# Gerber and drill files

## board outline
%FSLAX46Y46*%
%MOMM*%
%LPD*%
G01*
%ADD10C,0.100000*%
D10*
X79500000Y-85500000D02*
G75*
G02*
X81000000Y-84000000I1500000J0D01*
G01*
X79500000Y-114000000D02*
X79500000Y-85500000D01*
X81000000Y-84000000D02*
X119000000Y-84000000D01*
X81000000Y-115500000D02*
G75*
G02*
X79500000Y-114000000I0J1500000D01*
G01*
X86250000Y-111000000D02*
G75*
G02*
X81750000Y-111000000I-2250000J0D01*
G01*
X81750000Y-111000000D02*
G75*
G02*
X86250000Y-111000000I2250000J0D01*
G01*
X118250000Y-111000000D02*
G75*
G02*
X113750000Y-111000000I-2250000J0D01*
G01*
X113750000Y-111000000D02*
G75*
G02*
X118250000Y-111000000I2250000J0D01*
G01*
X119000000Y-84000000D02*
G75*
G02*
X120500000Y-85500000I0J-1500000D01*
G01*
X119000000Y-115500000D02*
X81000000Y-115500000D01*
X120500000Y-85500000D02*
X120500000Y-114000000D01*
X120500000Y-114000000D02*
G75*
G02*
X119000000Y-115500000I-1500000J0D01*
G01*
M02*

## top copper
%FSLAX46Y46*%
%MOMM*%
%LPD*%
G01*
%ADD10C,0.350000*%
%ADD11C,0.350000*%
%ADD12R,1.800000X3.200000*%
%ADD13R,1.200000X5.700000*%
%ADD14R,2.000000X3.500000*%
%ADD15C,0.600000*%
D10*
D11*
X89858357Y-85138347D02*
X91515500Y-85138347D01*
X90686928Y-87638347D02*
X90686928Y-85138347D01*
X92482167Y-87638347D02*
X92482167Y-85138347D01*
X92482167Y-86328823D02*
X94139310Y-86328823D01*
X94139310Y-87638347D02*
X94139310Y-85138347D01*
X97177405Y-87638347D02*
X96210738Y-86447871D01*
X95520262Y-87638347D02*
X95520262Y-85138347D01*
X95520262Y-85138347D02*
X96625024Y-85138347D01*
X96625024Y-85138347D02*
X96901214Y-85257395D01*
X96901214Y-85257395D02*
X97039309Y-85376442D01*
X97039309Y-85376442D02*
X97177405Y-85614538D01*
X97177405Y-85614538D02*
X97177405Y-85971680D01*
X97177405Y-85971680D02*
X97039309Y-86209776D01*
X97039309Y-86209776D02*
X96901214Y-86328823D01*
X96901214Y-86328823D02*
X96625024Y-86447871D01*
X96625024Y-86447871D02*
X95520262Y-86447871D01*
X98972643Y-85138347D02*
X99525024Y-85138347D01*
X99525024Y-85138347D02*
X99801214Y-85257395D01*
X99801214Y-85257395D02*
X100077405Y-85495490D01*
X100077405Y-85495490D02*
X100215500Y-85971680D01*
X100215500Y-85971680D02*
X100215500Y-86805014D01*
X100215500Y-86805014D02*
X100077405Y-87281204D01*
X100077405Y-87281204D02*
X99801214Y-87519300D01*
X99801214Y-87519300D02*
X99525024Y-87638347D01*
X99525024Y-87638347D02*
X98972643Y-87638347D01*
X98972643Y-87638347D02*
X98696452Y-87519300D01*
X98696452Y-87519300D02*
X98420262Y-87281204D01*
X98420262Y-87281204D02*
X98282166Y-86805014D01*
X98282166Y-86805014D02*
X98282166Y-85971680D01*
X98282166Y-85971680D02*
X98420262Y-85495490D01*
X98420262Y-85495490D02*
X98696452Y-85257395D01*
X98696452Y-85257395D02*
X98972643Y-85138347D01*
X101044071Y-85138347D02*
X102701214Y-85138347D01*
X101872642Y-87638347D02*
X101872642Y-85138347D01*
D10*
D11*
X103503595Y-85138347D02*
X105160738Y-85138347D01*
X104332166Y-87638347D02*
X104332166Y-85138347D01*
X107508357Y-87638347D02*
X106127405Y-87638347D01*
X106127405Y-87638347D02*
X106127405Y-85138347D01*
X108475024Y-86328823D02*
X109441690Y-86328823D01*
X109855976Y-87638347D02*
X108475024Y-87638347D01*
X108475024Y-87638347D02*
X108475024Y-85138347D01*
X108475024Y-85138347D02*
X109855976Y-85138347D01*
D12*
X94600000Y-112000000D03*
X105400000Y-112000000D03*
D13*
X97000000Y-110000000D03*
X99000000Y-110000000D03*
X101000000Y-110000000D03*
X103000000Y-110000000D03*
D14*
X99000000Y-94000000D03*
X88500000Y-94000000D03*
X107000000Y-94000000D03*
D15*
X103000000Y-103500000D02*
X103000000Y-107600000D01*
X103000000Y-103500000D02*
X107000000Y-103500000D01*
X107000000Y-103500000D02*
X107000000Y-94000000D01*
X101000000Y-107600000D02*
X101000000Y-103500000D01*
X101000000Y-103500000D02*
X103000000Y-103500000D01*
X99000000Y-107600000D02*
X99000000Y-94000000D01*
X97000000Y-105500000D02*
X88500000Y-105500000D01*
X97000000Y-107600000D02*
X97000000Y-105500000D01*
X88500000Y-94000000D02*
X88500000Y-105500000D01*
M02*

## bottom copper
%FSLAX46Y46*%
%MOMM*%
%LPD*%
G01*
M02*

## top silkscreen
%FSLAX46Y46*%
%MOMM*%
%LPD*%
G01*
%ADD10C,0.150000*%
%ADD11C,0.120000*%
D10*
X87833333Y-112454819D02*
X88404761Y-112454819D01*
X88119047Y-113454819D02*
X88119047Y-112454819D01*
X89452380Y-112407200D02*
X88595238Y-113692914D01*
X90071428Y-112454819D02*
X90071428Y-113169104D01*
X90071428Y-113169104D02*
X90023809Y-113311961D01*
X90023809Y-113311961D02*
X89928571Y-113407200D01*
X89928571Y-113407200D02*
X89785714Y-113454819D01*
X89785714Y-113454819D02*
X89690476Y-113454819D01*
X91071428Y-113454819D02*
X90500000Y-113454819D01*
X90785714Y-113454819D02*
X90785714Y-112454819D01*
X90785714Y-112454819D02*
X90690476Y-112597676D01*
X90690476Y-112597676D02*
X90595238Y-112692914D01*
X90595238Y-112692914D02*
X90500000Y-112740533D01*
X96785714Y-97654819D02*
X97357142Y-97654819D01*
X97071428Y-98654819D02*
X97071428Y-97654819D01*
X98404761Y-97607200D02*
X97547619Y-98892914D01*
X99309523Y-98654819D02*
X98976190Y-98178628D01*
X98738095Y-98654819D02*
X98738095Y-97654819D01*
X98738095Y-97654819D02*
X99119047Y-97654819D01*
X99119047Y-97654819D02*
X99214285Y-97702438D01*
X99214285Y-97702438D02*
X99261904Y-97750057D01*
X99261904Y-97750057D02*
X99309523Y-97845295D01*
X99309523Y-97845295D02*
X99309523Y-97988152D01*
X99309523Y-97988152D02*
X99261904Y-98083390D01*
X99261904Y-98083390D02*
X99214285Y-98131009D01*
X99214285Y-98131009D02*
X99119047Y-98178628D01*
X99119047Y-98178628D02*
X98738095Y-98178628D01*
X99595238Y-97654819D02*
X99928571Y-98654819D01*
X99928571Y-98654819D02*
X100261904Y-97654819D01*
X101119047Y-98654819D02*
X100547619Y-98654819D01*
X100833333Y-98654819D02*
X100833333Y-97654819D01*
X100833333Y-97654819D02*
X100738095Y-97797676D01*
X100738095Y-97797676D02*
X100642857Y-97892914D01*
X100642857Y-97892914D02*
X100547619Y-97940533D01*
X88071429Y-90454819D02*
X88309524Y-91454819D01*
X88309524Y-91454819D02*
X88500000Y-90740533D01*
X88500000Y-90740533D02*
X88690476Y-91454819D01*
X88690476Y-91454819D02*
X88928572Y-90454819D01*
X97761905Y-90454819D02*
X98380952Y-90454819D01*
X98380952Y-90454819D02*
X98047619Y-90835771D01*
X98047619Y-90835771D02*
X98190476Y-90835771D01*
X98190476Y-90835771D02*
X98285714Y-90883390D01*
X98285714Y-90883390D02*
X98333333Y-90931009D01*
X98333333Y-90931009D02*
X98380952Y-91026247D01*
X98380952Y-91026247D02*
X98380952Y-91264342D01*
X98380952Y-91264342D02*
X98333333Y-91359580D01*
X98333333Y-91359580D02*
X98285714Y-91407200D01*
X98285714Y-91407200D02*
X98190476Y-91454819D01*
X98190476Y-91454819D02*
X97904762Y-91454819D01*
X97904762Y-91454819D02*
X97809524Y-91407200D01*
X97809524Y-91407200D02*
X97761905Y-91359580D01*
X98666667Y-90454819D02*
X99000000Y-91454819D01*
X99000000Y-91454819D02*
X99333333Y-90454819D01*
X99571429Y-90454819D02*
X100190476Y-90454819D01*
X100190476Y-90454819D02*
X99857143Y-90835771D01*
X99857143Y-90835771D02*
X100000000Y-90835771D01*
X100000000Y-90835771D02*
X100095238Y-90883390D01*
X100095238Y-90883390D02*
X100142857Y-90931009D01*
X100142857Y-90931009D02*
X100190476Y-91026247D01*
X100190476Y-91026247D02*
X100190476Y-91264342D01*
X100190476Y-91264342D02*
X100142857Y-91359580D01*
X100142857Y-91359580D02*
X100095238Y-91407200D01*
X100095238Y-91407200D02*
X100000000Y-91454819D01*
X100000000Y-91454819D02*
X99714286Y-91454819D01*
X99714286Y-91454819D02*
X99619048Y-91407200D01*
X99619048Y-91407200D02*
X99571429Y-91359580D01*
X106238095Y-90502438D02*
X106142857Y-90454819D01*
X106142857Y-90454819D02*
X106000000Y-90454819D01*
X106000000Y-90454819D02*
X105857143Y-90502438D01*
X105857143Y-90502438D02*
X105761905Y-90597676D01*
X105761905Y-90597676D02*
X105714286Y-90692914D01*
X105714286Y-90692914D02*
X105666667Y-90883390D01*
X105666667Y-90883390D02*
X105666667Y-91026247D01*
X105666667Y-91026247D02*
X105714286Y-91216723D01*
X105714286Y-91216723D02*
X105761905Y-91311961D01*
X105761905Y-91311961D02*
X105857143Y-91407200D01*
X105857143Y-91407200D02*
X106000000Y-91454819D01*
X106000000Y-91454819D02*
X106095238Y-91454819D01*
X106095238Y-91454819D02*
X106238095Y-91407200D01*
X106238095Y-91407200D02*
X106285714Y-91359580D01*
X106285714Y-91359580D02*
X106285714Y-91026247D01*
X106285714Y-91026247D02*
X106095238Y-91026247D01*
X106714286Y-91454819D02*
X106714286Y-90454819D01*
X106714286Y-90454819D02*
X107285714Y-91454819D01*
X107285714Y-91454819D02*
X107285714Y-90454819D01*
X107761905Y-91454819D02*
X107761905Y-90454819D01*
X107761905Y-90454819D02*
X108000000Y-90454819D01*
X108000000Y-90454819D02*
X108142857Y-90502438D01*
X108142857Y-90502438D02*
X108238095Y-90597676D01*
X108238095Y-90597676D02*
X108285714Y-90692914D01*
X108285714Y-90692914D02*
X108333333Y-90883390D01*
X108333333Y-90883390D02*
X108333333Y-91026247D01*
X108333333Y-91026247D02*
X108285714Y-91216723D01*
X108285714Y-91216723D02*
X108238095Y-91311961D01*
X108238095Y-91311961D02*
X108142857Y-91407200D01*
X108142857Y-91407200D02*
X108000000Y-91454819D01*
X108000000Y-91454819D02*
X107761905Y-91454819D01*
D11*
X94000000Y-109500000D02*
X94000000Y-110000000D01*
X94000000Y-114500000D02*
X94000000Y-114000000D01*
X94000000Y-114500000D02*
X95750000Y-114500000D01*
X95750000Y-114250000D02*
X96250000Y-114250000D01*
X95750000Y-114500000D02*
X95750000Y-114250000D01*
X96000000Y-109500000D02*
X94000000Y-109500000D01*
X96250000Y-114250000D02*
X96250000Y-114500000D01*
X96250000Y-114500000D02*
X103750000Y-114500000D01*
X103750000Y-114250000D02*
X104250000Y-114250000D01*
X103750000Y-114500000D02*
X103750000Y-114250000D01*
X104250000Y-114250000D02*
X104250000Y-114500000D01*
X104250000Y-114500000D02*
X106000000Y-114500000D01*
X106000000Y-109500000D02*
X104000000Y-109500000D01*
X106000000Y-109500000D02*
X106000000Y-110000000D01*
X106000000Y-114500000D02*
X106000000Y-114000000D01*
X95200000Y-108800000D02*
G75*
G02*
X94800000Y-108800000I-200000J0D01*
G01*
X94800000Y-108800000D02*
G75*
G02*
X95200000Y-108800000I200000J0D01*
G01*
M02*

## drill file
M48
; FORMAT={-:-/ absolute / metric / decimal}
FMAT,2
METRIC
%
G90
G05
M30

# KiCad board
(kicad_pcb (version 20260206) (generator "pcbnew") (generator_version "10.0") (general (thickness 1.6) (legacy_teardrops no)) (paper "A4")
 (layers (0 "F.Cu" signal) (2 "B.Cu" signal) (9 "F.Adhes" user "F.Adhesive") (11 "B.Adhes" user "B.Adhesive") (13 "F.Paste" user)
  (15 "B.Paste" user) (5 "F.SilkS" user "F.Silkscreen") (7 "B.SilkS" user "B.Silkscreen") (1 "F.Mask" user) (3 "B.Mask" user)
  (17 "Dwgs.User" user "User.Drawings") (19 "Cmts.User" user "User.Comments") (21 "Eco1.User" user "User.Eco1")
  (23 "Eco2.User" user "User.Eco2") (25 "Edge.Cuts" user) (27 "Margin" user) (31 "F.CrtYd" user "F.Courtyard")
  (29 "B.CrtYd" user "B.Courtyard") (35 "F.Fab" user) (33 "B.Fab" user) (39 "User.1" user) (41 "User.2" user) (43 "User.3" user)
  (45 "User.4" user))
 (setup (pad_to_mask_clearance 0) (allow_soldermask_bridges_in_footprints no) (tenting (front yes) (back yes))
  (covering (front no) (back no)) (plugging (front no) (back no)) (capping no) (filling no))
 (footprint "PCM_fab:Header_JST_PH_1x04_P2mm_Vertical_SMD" (layer "F.Cu") (at 98 110 90)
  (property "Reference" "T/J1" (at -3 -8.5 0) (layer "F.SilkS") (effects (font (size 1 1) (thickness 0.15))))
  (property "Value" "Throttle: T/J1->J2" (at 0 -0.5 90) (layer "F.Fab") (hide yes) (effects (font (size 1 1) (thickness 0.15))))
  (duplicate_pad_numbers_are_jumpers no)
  (fp_line (start 0.5 -4) (end 0 -4) (stroke (width 0.12) (type solid)) (layer "F.SilkS"))
  (fp_line (start -4.5 -4) (end -4 -4) (stroke (width 0.12) (type solid)) (layer "F.SilkS"))
  (fp_line (start -4.5 -4) (end -4.5 -2.25) (stroke (width 0.12) (type solid)) (layer "F.SilkS"))
  (fp_line (start -4.25 -2.25) (end -4.25 -1.75) (stroke (width 0.12) (type solid)) (layer "F.SilkS"))
  (fp_line (start -4.5 -2.25) (end -4.25 -2.25) (stroke (width 0.12) (type solid)) (layer "F.SilkS"))
  (fp_line (start 0.5 -2) (end 0.5 -4) (stroke (width 0.12) (type solid)) (layer "F.SilkS"))
  (fp_line (start -4.25 -1.75) (end -4.5 -1.75) (stroke (width 0.12) (type solid)) (layer "F.SilkS"))
  (fp_line (start -4.5 -1.75) (end -4.5 5.75) (stroke (width 0.12) (type solid)) (layer "F.SilkS"))
  (fp_line (start -4.25 5.75) (end -4.25 6.25) (stroke (width 0.12) (type solid)) (layer "F.SilkS"))
  (fp_line (start -4.5 5.75) (end -4.25 5.75) (stroke (width 0.12) (type solid)) (layer "F.SilkS"))
  (fp_line (start -4.25 6.25) (end -4.5 6.25) (stroke (width 0.12) (type solid)) (layer "F.SilkS"))
  (fp_line (start -4.5 6.25) (end -4.5 8) (stroke (width 0.12) (type solid)) (layer "F.SilkS"))
  (fp_line (start 0.5 8) (end 0.5 6) (stroke (width 0.12) (type solid)) (layer "F.SilkS"))
  (fp_line (start 0.5 8) (end 0 8) (stroke (width 0.12) (type solid)) (layer "F.SilkS"))
  (fp_line (start -4.5 8) (end -4 8) (stroke (width 0.12) (type solid)) (layer "F.SilkS"))
  (fp_circle (center 1.2 -3) (end 1.4 -3) (stroke (width 0.12) (type solid)) (fill no) (layer "F.SilkS"))
  (pad "" smd rect (at -2 -3.4 90) (size 3.2 1.8) (layers "F.Cu" "F.Mask" "F.Paste"))
  (pad "" smd rect (at -2 7.4 90) (size 3.2 1.8) (layers "F.Cu" "F.Mask" "F.Paste"))
  (pad "1" smd rect (at 0 -1 90) (size 5.7 1.2) (layers "F.Cu" "F.Mask" "F.Paste") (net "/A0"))
  (pad "2" smd rect (at 0 1 90) (size 5.7 1.2) (layers "F.Cu" "F.Mask" "F.Paste") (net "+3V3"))
  (pad "3" smd rect (at 0 3 90) (size 5.7 1.2) (layers "F.Cu" "F.Mask" "F.Paste") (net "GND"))
  (pad "4" smd rect (at 0 5 90) (size 5.7 1.2) (layers "F.Cu" "F.Mask" "F.Paste") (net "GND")))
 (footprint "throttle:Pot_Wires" (layer "F.Cu") (at 99 94)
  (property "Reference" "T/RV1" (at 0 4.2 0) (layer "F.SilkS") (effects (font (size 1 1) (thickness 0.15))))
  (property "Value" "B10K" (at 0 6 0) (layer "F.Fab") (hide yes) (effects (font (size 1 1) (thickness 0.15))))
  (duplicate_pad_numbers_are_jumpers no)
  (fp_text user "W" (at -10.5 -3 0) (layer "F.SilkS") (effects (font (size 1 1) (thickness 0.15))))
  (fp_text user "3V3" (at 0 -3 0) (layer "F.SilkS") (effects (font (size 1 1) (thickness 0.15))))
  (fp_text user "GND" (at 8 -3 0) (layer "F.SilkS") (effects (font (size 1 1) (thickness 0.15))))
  (pad "1" smd rect (at 0 0) (size 2 3.5) (layers "F.Cu" "F.Mask") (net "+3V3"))
  (pad "2" smd rect (at -10.5 0) (size 2 3.5) (layers "F.Cu" "F.Mask") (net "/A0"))
  (pad "3" smd rect (at 8 0) (size 2 3.5) (layers "F.Cu" "F.Mask") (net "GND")))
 (gr_arc (start 79.5 85.5) (mid 79.939339 84.439339) (end 81 84) (stroke (width 0.1) (type default)) (layer "Edge.Cuts"))
 (gr_line (start 79.5 114) (end 79.5 85.5) (stroke (width 0.1) (type default)) (layer "Edge.Cuts"))
 (gr_line (start 81 84) (end 119 84) (stroke (width 0.1) (type default)) (layer "Edge.Cuts"))
 (gr_arc (start 81 115.5) (mid 79.939339 115.06066) (end 79.5 114) (stroke (width 0.1) (type default)) (layer "Edge.Cuts"))
 (gr_circle (center 84 111) (end 86.25 111) (stroke (width 0.1) (type default)) (fill no) (layer "Edge.Cuts"))
 (gr_circle (center 116 111) (end 118.25 111) (stroke (width 0.1) (type default)) (fill no) (layer "Edge.Cuts"))
 (gr_arc (start 119 84) (mid 120.06066 84.439339) (end 120.5 85.5) (stroke (width 0.1) (type default)) (layer "Edge.Cuts"))
 (gr_line (start 119 115.5) (end 81 115.5) (stroke (width 0.1) (type default)) (layer "Edge.Cuts"))
 (gr_line (start 120.5 85.5) (end 120.5 114) (stroke (width 0.1) (type default)) (layer "Edge.Cuts"))
 (gr_arc (start 120.5 114) (mid 120.06066 115.06066) (end 119 115.5) (stroke (width 0.1) (type default)) (layer "Edge.Cuts"))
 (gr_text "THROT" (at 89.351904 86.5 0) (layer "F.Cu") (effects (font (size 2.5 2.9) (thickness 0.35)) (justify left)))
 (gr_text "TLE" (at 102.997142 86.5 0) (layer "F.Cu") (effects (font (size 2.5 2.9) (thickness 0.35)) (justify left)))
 (segment (start 103 103.5) (end 103 107.6) (width 0.6) (layer "F.Cu") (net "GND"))
 (segment (start 103 103.5) (end 107 103.5) (width 0.6) (layer "F.Cu") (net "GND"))
 (segment (start 107 103.5) (end 107 94) (width 0.6) (layer "F.Cu") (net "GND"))
 (segment (start 101 107.6) (end 101 103.5) (width 0.6) (layer "F.Cu") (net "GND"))
 (segment (start 101 103.5) (end 103 103.5) (width 0.6) (layer "F.Cu") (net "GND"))
 (segment (start 99 107.6) (end 99 94) (width 0.6) (layer "F.Cu") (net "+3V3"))
 (segment (start 97 105.5) (end 88.5 105.5) (width 0.6) (layer "F.Cu") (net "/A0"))
 (segment (start 97 107.6) (end 97 105.5) (width 0.6) (layer "F.Cu") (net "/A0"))
 (segment (start 88.5 94) (end 88.5 105.5) (width 0.6) (layer "F.Cu") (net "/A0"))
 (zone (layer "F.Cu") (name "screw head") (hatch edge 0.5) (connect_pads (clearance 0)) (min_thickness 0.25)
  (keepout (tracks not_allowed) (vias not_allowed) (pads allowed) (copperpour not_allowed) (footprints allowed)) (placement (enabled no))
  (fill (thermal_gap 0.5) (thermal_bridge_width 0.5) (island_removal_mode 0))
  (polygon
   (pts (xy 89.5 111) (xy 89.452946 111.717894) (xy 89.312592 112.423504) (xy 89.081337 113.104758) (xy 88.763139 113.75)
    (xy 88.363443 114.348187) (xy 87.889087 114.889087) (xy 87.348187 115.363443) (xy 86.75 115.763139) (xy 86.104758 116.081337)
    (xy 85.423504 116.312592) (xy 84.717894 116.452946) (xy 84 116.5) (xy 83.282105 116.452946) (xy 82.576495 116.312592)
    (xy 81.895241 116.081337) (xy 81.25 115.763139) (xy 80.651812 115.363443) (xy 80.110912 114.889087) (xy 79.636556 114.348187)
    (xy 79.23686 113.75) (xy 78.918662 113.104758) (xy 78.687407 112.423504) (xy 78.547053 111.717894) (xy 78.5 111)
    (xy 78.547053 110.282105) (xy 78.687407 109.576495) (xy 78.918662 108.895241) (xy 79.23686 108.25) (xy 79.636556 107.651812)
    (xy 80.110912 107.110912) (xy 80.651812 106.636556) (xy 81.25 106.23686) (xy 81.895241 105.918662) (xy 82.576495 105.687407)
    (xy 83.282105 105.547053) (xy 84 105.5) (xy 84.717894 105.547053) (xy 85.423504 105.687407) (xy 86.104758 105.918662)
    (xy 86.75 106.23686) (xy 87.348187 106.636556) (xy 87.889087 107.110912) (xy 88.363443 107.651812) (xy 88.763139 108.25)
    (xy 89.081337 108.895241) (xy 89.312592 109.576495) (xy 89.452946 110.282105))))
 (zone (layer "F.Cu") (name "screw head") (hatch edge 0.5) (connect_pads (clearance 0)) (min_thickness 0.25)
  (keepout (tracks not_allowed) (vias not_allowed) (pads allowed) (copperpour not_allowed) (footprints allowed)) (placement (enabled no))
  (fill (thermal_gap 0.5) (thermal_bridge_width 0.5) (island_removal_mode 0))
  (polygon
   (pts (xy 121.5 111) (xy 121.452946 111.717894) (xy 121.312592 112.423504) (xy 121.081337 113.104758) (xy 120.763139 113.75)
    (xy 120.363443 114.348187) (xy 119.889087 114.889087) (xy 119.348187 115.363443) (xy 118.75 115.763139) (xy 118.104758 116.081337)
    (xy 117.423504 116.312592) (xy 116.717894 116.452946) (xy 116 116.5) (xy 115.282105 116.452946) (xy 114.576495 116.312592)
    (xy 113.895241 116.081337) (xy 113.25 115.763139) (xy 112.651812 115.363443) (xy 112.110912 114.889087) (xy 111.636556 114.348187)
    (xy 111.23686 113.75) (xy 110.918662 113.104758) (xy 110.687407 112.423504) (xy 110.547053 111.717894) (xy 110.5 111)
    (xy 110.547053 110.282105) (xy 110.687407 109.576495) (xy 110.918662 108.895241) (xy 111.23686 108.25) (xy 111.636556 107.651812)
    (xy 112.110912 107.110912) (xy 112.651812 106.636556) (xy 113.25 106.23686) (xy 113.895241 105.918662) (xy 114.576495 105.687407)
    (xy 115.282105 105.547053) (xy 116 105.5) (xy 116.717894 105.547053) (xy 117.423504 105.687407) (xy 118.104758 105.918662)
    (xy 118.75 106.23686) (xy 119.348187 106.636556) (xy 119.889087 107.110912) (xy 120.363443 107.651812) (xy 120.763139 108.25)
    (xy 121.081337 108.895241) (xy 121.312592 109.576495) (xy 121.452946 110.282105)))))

